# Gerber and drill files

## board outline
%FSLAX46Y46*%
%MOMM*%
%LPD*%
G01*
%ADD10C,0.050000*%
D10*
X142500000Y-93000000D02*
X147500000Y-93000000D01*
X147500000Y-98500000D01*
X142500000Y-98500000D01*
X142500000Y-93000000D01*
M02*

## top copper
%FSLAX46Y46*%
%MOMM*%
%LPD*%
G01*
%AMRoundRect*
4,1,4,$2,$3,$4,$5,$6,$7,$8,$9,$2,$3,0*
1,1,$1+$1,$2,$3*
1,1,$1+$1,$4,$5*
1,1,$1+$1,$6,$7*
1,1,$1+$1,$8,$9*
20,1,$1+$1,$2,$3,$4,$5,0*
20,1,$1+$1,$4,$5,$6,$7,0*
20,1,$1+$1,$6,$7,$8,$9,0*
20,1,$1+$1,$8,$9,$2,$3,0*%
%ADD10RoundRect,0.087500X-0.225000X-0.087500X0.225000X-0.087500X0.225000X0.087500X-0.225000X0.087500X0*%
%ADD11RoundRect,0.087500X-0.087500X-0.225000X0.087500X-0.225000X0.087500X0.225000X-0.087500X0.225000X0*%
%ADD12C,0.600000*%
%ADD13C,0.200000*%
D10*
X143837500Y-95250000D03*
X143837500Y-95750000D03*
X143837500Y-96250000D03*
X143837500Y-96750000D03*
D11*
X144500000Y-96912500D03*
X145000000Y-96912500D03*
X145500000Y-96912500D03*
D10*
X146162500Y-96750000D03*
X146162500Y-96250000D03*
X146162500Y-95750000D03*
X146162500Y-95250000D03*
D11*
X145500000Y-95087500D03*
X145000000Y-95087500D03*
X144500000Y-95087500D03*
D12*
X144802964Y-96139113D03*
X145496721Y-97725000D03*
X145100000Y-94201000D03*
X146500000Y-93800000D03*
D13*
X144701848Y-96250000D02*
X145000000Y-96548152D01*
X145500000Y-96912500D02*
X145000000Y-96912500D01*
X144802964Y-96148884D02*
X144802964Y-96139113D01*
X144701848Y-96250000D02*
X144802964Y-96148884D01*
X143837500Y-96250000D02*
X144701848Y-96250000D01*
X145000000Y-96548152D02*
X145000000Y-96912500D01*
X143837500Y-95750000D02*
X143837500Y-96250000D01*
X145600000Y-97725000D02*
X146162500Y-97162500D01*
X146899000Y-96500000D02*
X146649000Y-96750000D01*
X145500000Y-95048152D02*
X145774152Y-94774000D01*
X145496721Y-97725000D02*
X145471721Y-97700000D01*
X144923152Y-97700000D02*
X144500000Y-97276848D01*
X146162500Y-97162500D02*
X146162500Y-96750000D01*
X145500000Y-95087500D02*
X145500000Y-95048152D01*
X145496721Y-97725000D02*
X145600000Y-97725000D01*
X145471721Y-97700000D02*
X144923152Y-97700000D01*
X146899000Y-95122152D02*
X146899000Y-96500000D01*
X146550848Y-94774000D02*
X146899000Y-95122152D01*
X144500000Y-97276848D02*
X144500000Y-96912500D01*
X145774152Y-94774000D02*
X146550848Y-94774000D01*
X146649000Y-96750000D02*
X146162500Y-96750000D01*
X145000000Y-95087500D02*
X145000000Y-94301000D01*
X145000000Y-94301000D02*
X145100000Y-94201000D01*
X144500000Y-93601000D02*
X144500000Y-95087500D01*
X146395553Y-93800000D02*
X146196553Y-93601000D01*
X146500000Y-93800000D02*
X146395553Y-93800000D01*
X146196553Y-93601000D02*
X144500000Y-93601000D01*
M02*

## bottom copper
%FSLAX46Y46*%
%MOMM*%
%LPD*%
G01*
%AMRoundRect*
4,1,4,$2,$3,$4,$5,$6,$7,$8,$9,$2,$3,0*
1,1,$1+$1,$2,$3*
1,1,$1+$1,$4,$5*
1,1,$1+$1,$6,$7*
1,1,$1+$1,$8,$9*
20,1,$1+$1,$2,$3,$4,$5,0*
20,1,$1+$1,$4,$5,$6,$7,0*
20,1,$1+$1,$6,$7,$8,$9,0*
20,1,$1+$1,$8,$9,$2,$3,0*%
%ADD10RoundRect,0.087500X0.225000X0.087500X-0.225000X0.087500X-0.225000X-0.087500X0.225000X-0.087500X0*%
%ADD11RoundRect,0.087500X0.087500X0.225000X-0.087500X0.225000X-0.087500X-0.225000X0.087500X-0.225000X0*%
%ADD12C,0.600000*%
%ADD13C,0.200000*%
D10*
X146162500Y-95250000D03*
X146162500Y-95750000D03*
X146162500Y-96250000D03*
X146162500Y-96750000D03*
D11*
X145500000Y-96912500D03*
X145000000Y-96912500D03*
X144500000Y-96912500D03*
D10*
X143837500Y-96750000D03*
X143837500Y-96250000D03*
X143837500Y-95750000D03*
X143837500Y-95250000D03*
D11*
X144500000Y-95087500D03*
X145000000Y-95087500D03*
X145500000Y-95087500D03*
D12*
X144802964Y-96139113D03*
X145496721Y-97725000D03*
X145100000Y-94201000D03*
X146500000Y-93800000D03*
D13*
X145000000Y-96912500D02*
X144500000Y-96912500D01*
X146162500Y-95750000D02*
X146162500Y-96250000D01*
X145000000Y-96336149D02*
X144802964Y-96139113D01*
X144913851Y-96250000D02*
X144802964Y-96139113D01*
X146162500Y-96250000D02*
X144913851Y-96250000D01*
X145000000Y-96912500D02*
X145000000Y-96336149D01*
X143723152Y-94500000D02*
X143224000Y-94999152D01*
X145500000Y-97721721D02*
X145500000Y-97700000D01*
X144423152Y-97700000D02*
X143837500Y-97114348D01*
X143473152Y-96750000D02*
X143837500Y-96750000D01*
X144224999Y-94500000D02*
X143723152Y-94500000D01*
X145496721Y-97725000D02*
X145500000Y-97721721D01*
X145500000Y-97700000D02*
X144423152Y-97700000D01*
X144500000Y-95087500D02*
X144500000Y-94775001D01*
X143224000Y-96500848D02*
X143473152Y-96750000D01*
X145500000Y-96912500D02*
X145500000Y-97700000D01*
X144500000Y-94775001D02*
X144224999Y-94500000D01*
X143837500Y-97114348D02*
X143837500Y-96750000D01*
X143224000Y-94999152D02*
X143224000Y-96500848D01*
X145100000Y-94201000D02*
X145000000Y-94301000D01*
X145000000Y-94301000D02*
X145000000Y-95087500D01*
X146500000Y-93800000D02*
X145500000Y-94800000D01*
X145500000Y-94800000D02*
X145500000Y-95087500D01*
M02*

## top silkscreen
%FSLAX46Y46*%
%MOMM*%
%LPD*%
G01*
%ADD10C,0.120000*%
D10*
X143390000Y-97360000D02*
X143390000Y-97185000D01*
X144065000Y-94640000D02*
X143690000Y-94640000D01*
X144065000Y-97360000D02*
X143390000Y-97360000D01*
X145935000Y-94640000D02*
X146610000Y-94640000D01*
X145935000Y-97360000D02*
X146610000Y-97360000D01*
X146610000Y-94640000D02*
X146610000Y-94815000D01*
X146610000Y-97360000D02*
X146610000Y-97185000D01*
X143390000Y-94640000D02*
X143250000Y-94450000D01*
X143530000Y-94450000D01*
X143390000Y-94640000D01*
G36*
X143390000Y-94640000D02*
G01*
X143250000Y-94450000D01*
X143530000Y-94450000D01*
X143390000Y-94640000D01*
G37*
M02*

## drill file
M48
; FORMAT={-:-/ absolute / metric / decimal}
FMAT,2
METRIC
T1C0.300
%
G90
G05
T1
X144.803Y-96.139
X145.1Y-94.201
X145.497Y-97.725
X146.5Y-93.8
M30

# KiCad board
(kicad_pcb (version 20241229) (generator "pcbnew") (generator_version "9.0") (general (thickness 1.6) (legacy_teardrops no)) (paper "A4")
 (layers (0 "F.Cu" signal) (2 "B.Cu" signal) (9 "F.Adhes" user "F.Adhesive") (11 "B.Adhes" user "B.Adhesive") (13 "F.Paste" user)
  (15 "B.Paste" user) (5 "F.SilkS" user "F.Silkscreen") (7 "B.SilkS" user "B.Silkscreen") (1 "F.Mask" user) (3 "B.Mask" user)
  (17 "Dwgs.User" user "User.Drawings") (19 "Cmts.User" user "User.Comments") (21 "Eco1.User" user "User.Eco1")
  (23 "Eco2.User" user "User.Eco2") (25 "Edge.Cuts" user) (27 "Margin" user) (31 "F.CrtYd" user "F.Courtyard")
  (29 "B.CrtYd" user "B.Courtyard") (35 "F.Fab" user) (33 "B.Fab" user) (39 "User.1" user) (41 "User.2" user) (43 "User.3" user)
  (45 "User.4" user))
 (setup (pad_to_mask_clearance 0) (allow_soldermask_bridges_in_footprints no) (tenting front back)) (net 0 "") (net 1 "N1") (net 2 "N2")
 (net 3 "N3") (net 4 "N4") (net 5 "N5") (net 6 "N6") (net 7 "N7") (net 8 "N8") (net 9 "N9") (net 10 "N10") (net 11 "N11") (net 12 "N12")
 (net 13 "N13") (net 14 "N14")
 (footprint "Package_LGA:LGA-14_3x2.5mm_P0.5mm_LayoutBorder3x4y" (layer "F.Cu") (at 145 96)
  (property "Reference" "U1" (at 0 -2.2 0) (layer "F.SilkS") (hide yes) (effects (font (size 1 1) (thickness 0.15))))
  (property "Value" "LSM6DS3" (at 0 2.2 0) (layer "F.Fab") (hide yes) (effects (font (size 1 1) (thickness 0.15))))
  (fp_line (start -1.61 1.36) (end -1.61 1.185) (stroke (width 0.12) (type solid)) (layer "F.SilkS"))
  (fp_line (start -0.935 -1.36) (end -1.31 -1.36) (stroke (width 0.12) (type solid)) (layer "F.SilkS"))
  (fp_line (start -0.935 1.36) (end -1.61 1.36) (stroke (width 0.12) (type solid)) (layer "F.SilkS"))
  (fp_line (start 0.935 -1.36) (end 1.61 -1.36) (stroke (width 0.12) (type solid)) (layer "F.SilkS"))
  (fp_line (start 0.935 1.36) (end 1.61 1.36) (stroke (width 0.12) (type solid)) (layer "F.SilkS"))
  (fp_line (start 1.61 -1.36) (end 1.61 -1.185) (stroke (width 0.12) (type solid)) (layer "F.SilkS"))
  (fp_line (start 1.61 1.36) (end 1.61 1.185) (stroke (width 0.12) (type solid)) (layer "F.SilkS"))
  (fp_poly
   (pts (xy -1.61 -1.36) (xy -1.75 -1.55) (xy -1.47 -1.55) (xy -1.61 -1.36)) (stroke (width 0.12) (type solid)) (fill yes) (layer "F.SilkS"))
  (pad "1" smd roundrect (at -1.1625 -0.75) (size 0.625 0.35) (layers "F.Cu" "F.Mask" "F.Paste") (roundrect_rratio 0.25) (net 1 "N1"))
  (pad "2" smd roundrect (at -1.1625 -0.25) (size 0.625 0.35) (layers "F.Cu" "F.Mask" "F.Paste") (roundrect_rratio 0.25) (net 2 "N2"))
  (pad "3" smd roundrect (at -1.1625 0.25) (size 0.625 0.35) (layers "F.Cu" "F.Mask" "F.Paste") (roundrect_rratio 0.25) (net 2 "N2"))
  (pad "4" smd roundrect (at -1.1625 0.75) (size 0.625 0.35) (layers "F.Cu" "F.Mask" "F.Paste") (roundrect_rratio 0.25) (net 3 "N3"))
  (pad "5" smd roundrect (at -0.5 0.9125) (size 0.35 0.625) (layers "F.Cu" "F.Mask" "F.Paste") (roundrect_rratio 0.25) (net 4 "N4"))
  (pad "6" smd roundrect (at 0 0.9125) (size 0.35 0.625) (layers "F.Cu" "F.Mask" "F.Paste") (roundrect_rratio 0.25) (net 2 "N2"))
  (pad "7" smd roundrect (at 0.5 0.9125) (size 0.35 0.625) (layers "F.Cu" "F.Mask" "F.Paste") (roundrect_rratio 0.25) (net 2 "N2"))
  (pad "8" smd roundrect (at 1.1625 0.75) (size 0.625 0.35) (layers "F.Cu" "F.Mask" "F.Paste") (roundrect_rratio 0.25) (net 4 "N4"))
  (pad "9" smd roundrect (at 1.1625 0.25) (size 0.625 0.35) (layers "F.Cu" "F.Mask" "F.Paste") (roundrect_rratio 0.25) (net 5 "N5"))
  (pad "10" smd roundrect (at 1.1625 -0.25) (size 0.625 0.35) (layers "F.Cu" "F.Mask" "F.Paste") (roundrect_rratio 0.25) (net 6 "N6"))
  (pad "11" smd roundrect (at 1.1625 -0.75) (size 0.625 0.35) (layers "F.Cu" "F.Mask" "F.Paste") (roundrect_rratio 0.25) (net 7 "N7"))
  (pad "12" smd roundrect (at 0.5 -0.9125) (size 0.35 0.625) (layers "F.Cu" "F.Mask" "F.Paste") (roundrect_rratio 0.25) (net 4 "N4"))
  (pad "13" smd roundrect (at 0 -0.9125) (size 0.35 0.625) (layers "F.Cu" "F.Mask" "F.Paste") (roundrect_rratio 0.25) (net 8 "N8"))
  (pad "14" smd roundrect (at -0.5 -0.9125) (size 0.35 0.625) (layers "F.Cu" "F.Mask" "F.Paste") (roundrect_rratio 0.25) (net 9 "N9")))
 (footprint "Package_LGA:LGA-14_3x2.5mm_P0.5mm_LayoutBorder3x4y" (layer "B.Cu") (at 145 96 180)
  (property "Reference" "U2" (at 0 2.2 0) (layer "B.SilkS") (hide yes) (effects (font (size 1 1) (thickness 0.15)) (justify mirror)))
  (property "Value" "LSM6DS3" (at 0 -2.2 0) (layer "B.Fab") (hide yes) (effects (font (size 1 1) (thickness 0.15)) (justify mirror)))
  (pad "1" smd roundrect (at -1.1625 0.75 180) (size 0.625 0.35) (layers "B.Cu" "B.Mask" "B.Paste") (roundrect_rratio 0.25) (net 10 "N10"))
  (pad "2" smd roundrect (at -1.1625 0.25 180) (size 0.625 0.35) (layers "B.Cu" "B.Mask" "B.Paste") (roundrect_rratio 0.25) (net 2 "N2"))
  (pad "3" smd roundrect (at -1.1625 -0.25 180) (size 0.625 0.35) (layers "B.Cu" "B.Mask" "B.Paste") (roundrect_rratio 0.25) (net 2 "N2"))
  (pad "4" smd roundrect (at -1.1625 -0.75 180) (size 0.625 0.35) (layers "B.Cu" "B.Mask" "B.Paste") (roundrect_rratio 0.25) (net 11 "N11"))
  (pad "5" smd roundrect (at -0.5 -0.9125 180) (size 0.35 0.625) (layers "B.Cu" "B.Mask" "B.Paste") (roundrect_rratio 0.25) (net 4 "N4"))
  (pad "6" smd roundrect (at 0 -0.9125 180) (size 0.35 0.625) (layers "B.Cu" "B.Mask" "B.Paste") (roundrect_rratio 0.25) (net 2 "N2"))
  (pad "7" smd roundrect (at 0.5 -0.9125 180) (size 0.35 0.625) (layers "B.Cu" "B.Mask" "B.Paste") (roundrect_rratio 0.25) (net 2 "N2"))
  (pad "8" smd roundrect (at 1.1625 -0.75 180) (size 0.625 0.35) (layers "B.Cu" "B.Mask" "B.Paste") (roundrect_rratio 0.25) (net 4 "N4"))
  (pad "9" smd roundrect (at 1.1625 -0.25 180) (size 0.625 0.35) (layers "B.Cu" "B.Mask" "B.Paste") (roundrect_rratio 0.25) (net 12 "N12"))
  (pad "10" smd roundrect (at 1.1625 0.25 180) (size 0.625 0.35) (layers "B.Cu" "B.Mask" "B.Paste") (roundrect_rratio 0.25) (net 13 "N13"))
  (pad "11" smd roundrect (at 1.1625 0.75 180) (size 0.625 0.35) (layers "B.Cu" "B.Mask" "B.Paste") (roundrect_rratio 0.25) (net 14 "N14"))
  (pad "12" smd roundrect (at 0.5 0.9125 180) (size 0.35 0.625) (layers "B.Cu" "B.Mask" "B.Paste") (roundrect_rratio 0.25) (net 4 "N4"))
  (pad "13" smd roundrect (at 0 0.9125 180) (size 0.35 0.625) (layers "B.Cu" "B.Mask" "B.Paste") (roundrect_rratio 0.25) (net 8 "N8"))
  (pad "14" smd roundrect (at -0.5 0.9125 180) (size 0.35 0.625) (layers "B.Cu" "B.Mask" "B.Paste") (roundrect_rratio 0.25) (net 9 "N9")))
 (gr_rect (start 142.5 93) (end 147.5 98.5) (stroke (width 0.05) (type default)) (fill no) (layer "Edge.Cuts"))
 (segment (start 144.701848 96.25) (end 145 96.548152) (width 0.2) (layer "F.Cu") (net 2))
 (segment (start 145.5 96.9125) (end 145 96.9125) (width 0.2) (layer "F.Cu") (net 2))
 (segment (start 144.802964 96.148884) (end 144.802964 96.139113) (width 0.2) (layer "F.Cu") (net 2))
 (segment (start 144.701848 96.25) (end 144.802964 96.148884) (width 0.2) (layer "F.Cu") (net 2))
 (segment (start 143.8375 96.25) (end 144.701848 96.25) (width 0.2) (layer "F.Cu") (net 2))
 (segment (start 145 96.548152) (end 145 96.9125) (width 0.2) (layer "F.Cu") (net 2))
 (segment (start 143.8375 95.75) (end 143.8375 96.25) (width 0.2) (layer "F.Cu") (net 2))
 (via (at 144.802964 96.139113) (size 0.6) (drill 0.3) (layers "F.Cu" "B.Cu") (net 2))
 (segment (start 145 96.9125) (end 144.5 96.9125) (width 0.2) (layer "B.Cu") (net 2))
 (segment (start 146.1625 95.75) (end 146.1625 96.25) (width 0.2) (layer "B.Cu") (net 2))
 (segment (start 145 96.336149) (end 144.802964 96.139113) (width 0.2) (layer "B.Cu") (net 2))
 (segment (start 144.913851 96.25) (end 144.802964 96.139113) (width 0.2) (layer "B.Cu") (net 2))
 (segment (start 146.1625 96.25) (end 144.913851 96.25) (width 0.2) (layer "B.Cu") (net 2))
 (segment (start 145 96.9125) (end 145 96.336149) (width 0.2) (layer "B.Cu") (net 2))
 (segment (start 145.6 97.725) (end 146.1625 97.1625) (width 0.2) (layer "F.Cu") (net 4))
 (segment (start 146.899 96.5) (end 146.649 96.75) (width 0.2) (layer "F.Cu") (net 4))
 (segment (start 145.5 95.048152) (end 145.774152 94.774) (width 0.2) (layer "F.Cu") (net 4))
 (segment (start 145.496721 97.725) (end 145.471721 97.7) (width 0.2) (layer "F.Cu") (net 4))
 (segment (start 144.923152 97.7) (end 144.5 97.276848) (width 0.2) (layer "F.Cu") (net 4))
 (segment (start 146.1625 97.1625) (end 146.1625 96.75) (width 0.2) (layer "F.Cu") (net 4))
 (segment (start 145.5 95.0875) (end 145.5 95.048152) (width 0.2) (layer "F.Cu") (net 4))
 (segment (start 145.496721 97.725) (end 145.6 97.725) (width 0.2) (layer "F.Cu") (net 4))
 (segment (start 145.471721 97.7) (end 144.923152 97.7) (width 0.2) (layer "F.Cu") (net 4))
 (segment (start 146.899 95.122152) (end 146.899 96.5) (width 0.2) (layer "F.Cu") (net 4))
 (segment (start 146.550848 94.774) (end 146.899 95.122152) (width 0.2) (layer "F.Cu") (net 4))
 (segment (start 144.5 97.276848) (end 144.5 96.9125) (width 0.2) (layer "F.Cu") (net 4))
 (segment (start 145.774152 94.774) (end 146.550848 94.774) (width 0.2) (layer "F.Cu") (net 4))
 (segment (start 146.649 96.75) (end 146.1625 96.75) (width 0.2) (layer "F.Cu") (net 4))
 (via (at 145.496721 97.725) (size 0.6) (drill 0.3) (layers "F.Cu" "B.Cu") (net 4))
 (segment (start 143.723152 94.5) (end 143.224 94.999152) (width 0.2) (layer "B.Cu") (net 4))
 (segment (start 145.5 97.721721) (end 145.5 97.7) (width 0.2) (layer "B.Cu") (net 4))
 (segment (start 144.423152 97.7) (end 143.8375 97.114348) (width 0.2) (layer "B.Cu") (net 4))
 (segment (start 143.473152 96.75) (end 143.8375 96.75) (width 0.2) (layer "B.Cu") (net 4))
 (segment (start 144.224999 94.5) (end 143.723152 94.5) (width 0.2) (layer "B.Cu") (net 4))
 (segment (start 145.496721 97.725) (end 145.5 97.721721) (width 0.2) (layer "B.Cu") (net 4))
 (segment (start 145.5 97.7) (end 144.423152 97.7) (width 0.2) (layer "B.Cu") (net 4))
 (segment (start 144.5 95.0875) (end 144.5 94.775001) (width 0.2) (layer "B.Cu") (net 4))
 (segment (start 143.224 96.500848) (end 143.473152 96.75) (width 0.2) (layer "B.Cu") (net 4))
 (segment (start 145.5 96.9125) (end 145.5 97.7) (width 0.2) (layer "B.Cu") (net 4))
 (segment (start 144.5 94.775001) (end 144.224999 94.5) (width 0.2) (layer "B.Cu") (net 4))
 (segment (start 143.8375 97.114348) (end 143.8375 96.75) (width 0.2) (layer "B.Cu") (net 4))
 (segment (start 143.224 94.999152) (end 143.224 96.500848) (width 0.2) (layer "B.Cu") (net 4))
 (segment (start 145 95.0875) (end 145 94.301) (width 0.2) (layer "F.Cu") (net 8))
 (segment (start 145 94.301) (end 145.1 94.201) (width 0.2) (layer "F.Cu") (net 8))
 (via (at 145.1 94.201) (size 0.6) (drill 0.3) (layers "F.Cu" "B.Cu") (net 8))
 (segment (start 145.1 94.201) (end 145 94.301) (width 0.2) (layer "B.Cu") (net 8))
 (segment (start 145 94.301) (end 145 95.0875) (width 0.2) (layer "B.Cu") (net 8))
 (segment (start 144.5 93.601) (end 144.5 95.0875) (width 0.2) (layer "F.Cu") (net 9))
 (segment (start 146.395553 93.8) (end 146.196553 93.601) (width 0.2) (layer "F.Cu") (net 9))
 (segment (start 146.5 93.8) (end 146.395553 93.8) (width 0.2) (layer "F.Cu") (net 9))
 (segment (start 146.196553 93.601) (end 144.5 93.601) (width 0.2) (layer "F.Cu") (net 9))
 (via (at 146.5 93.8) (size 0.6) (drill 0.3) (layers "F.Cu" "B.Cu") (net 9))
 (segment (start 146.5 93.8) (end 145.5 94.8) (width 0.2) (layer "B.Cu") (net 9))
 (segment (start 145.5 94.8) (end 145.5 95.0875) (width 0.2) (layer "B.Cu") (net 9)))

